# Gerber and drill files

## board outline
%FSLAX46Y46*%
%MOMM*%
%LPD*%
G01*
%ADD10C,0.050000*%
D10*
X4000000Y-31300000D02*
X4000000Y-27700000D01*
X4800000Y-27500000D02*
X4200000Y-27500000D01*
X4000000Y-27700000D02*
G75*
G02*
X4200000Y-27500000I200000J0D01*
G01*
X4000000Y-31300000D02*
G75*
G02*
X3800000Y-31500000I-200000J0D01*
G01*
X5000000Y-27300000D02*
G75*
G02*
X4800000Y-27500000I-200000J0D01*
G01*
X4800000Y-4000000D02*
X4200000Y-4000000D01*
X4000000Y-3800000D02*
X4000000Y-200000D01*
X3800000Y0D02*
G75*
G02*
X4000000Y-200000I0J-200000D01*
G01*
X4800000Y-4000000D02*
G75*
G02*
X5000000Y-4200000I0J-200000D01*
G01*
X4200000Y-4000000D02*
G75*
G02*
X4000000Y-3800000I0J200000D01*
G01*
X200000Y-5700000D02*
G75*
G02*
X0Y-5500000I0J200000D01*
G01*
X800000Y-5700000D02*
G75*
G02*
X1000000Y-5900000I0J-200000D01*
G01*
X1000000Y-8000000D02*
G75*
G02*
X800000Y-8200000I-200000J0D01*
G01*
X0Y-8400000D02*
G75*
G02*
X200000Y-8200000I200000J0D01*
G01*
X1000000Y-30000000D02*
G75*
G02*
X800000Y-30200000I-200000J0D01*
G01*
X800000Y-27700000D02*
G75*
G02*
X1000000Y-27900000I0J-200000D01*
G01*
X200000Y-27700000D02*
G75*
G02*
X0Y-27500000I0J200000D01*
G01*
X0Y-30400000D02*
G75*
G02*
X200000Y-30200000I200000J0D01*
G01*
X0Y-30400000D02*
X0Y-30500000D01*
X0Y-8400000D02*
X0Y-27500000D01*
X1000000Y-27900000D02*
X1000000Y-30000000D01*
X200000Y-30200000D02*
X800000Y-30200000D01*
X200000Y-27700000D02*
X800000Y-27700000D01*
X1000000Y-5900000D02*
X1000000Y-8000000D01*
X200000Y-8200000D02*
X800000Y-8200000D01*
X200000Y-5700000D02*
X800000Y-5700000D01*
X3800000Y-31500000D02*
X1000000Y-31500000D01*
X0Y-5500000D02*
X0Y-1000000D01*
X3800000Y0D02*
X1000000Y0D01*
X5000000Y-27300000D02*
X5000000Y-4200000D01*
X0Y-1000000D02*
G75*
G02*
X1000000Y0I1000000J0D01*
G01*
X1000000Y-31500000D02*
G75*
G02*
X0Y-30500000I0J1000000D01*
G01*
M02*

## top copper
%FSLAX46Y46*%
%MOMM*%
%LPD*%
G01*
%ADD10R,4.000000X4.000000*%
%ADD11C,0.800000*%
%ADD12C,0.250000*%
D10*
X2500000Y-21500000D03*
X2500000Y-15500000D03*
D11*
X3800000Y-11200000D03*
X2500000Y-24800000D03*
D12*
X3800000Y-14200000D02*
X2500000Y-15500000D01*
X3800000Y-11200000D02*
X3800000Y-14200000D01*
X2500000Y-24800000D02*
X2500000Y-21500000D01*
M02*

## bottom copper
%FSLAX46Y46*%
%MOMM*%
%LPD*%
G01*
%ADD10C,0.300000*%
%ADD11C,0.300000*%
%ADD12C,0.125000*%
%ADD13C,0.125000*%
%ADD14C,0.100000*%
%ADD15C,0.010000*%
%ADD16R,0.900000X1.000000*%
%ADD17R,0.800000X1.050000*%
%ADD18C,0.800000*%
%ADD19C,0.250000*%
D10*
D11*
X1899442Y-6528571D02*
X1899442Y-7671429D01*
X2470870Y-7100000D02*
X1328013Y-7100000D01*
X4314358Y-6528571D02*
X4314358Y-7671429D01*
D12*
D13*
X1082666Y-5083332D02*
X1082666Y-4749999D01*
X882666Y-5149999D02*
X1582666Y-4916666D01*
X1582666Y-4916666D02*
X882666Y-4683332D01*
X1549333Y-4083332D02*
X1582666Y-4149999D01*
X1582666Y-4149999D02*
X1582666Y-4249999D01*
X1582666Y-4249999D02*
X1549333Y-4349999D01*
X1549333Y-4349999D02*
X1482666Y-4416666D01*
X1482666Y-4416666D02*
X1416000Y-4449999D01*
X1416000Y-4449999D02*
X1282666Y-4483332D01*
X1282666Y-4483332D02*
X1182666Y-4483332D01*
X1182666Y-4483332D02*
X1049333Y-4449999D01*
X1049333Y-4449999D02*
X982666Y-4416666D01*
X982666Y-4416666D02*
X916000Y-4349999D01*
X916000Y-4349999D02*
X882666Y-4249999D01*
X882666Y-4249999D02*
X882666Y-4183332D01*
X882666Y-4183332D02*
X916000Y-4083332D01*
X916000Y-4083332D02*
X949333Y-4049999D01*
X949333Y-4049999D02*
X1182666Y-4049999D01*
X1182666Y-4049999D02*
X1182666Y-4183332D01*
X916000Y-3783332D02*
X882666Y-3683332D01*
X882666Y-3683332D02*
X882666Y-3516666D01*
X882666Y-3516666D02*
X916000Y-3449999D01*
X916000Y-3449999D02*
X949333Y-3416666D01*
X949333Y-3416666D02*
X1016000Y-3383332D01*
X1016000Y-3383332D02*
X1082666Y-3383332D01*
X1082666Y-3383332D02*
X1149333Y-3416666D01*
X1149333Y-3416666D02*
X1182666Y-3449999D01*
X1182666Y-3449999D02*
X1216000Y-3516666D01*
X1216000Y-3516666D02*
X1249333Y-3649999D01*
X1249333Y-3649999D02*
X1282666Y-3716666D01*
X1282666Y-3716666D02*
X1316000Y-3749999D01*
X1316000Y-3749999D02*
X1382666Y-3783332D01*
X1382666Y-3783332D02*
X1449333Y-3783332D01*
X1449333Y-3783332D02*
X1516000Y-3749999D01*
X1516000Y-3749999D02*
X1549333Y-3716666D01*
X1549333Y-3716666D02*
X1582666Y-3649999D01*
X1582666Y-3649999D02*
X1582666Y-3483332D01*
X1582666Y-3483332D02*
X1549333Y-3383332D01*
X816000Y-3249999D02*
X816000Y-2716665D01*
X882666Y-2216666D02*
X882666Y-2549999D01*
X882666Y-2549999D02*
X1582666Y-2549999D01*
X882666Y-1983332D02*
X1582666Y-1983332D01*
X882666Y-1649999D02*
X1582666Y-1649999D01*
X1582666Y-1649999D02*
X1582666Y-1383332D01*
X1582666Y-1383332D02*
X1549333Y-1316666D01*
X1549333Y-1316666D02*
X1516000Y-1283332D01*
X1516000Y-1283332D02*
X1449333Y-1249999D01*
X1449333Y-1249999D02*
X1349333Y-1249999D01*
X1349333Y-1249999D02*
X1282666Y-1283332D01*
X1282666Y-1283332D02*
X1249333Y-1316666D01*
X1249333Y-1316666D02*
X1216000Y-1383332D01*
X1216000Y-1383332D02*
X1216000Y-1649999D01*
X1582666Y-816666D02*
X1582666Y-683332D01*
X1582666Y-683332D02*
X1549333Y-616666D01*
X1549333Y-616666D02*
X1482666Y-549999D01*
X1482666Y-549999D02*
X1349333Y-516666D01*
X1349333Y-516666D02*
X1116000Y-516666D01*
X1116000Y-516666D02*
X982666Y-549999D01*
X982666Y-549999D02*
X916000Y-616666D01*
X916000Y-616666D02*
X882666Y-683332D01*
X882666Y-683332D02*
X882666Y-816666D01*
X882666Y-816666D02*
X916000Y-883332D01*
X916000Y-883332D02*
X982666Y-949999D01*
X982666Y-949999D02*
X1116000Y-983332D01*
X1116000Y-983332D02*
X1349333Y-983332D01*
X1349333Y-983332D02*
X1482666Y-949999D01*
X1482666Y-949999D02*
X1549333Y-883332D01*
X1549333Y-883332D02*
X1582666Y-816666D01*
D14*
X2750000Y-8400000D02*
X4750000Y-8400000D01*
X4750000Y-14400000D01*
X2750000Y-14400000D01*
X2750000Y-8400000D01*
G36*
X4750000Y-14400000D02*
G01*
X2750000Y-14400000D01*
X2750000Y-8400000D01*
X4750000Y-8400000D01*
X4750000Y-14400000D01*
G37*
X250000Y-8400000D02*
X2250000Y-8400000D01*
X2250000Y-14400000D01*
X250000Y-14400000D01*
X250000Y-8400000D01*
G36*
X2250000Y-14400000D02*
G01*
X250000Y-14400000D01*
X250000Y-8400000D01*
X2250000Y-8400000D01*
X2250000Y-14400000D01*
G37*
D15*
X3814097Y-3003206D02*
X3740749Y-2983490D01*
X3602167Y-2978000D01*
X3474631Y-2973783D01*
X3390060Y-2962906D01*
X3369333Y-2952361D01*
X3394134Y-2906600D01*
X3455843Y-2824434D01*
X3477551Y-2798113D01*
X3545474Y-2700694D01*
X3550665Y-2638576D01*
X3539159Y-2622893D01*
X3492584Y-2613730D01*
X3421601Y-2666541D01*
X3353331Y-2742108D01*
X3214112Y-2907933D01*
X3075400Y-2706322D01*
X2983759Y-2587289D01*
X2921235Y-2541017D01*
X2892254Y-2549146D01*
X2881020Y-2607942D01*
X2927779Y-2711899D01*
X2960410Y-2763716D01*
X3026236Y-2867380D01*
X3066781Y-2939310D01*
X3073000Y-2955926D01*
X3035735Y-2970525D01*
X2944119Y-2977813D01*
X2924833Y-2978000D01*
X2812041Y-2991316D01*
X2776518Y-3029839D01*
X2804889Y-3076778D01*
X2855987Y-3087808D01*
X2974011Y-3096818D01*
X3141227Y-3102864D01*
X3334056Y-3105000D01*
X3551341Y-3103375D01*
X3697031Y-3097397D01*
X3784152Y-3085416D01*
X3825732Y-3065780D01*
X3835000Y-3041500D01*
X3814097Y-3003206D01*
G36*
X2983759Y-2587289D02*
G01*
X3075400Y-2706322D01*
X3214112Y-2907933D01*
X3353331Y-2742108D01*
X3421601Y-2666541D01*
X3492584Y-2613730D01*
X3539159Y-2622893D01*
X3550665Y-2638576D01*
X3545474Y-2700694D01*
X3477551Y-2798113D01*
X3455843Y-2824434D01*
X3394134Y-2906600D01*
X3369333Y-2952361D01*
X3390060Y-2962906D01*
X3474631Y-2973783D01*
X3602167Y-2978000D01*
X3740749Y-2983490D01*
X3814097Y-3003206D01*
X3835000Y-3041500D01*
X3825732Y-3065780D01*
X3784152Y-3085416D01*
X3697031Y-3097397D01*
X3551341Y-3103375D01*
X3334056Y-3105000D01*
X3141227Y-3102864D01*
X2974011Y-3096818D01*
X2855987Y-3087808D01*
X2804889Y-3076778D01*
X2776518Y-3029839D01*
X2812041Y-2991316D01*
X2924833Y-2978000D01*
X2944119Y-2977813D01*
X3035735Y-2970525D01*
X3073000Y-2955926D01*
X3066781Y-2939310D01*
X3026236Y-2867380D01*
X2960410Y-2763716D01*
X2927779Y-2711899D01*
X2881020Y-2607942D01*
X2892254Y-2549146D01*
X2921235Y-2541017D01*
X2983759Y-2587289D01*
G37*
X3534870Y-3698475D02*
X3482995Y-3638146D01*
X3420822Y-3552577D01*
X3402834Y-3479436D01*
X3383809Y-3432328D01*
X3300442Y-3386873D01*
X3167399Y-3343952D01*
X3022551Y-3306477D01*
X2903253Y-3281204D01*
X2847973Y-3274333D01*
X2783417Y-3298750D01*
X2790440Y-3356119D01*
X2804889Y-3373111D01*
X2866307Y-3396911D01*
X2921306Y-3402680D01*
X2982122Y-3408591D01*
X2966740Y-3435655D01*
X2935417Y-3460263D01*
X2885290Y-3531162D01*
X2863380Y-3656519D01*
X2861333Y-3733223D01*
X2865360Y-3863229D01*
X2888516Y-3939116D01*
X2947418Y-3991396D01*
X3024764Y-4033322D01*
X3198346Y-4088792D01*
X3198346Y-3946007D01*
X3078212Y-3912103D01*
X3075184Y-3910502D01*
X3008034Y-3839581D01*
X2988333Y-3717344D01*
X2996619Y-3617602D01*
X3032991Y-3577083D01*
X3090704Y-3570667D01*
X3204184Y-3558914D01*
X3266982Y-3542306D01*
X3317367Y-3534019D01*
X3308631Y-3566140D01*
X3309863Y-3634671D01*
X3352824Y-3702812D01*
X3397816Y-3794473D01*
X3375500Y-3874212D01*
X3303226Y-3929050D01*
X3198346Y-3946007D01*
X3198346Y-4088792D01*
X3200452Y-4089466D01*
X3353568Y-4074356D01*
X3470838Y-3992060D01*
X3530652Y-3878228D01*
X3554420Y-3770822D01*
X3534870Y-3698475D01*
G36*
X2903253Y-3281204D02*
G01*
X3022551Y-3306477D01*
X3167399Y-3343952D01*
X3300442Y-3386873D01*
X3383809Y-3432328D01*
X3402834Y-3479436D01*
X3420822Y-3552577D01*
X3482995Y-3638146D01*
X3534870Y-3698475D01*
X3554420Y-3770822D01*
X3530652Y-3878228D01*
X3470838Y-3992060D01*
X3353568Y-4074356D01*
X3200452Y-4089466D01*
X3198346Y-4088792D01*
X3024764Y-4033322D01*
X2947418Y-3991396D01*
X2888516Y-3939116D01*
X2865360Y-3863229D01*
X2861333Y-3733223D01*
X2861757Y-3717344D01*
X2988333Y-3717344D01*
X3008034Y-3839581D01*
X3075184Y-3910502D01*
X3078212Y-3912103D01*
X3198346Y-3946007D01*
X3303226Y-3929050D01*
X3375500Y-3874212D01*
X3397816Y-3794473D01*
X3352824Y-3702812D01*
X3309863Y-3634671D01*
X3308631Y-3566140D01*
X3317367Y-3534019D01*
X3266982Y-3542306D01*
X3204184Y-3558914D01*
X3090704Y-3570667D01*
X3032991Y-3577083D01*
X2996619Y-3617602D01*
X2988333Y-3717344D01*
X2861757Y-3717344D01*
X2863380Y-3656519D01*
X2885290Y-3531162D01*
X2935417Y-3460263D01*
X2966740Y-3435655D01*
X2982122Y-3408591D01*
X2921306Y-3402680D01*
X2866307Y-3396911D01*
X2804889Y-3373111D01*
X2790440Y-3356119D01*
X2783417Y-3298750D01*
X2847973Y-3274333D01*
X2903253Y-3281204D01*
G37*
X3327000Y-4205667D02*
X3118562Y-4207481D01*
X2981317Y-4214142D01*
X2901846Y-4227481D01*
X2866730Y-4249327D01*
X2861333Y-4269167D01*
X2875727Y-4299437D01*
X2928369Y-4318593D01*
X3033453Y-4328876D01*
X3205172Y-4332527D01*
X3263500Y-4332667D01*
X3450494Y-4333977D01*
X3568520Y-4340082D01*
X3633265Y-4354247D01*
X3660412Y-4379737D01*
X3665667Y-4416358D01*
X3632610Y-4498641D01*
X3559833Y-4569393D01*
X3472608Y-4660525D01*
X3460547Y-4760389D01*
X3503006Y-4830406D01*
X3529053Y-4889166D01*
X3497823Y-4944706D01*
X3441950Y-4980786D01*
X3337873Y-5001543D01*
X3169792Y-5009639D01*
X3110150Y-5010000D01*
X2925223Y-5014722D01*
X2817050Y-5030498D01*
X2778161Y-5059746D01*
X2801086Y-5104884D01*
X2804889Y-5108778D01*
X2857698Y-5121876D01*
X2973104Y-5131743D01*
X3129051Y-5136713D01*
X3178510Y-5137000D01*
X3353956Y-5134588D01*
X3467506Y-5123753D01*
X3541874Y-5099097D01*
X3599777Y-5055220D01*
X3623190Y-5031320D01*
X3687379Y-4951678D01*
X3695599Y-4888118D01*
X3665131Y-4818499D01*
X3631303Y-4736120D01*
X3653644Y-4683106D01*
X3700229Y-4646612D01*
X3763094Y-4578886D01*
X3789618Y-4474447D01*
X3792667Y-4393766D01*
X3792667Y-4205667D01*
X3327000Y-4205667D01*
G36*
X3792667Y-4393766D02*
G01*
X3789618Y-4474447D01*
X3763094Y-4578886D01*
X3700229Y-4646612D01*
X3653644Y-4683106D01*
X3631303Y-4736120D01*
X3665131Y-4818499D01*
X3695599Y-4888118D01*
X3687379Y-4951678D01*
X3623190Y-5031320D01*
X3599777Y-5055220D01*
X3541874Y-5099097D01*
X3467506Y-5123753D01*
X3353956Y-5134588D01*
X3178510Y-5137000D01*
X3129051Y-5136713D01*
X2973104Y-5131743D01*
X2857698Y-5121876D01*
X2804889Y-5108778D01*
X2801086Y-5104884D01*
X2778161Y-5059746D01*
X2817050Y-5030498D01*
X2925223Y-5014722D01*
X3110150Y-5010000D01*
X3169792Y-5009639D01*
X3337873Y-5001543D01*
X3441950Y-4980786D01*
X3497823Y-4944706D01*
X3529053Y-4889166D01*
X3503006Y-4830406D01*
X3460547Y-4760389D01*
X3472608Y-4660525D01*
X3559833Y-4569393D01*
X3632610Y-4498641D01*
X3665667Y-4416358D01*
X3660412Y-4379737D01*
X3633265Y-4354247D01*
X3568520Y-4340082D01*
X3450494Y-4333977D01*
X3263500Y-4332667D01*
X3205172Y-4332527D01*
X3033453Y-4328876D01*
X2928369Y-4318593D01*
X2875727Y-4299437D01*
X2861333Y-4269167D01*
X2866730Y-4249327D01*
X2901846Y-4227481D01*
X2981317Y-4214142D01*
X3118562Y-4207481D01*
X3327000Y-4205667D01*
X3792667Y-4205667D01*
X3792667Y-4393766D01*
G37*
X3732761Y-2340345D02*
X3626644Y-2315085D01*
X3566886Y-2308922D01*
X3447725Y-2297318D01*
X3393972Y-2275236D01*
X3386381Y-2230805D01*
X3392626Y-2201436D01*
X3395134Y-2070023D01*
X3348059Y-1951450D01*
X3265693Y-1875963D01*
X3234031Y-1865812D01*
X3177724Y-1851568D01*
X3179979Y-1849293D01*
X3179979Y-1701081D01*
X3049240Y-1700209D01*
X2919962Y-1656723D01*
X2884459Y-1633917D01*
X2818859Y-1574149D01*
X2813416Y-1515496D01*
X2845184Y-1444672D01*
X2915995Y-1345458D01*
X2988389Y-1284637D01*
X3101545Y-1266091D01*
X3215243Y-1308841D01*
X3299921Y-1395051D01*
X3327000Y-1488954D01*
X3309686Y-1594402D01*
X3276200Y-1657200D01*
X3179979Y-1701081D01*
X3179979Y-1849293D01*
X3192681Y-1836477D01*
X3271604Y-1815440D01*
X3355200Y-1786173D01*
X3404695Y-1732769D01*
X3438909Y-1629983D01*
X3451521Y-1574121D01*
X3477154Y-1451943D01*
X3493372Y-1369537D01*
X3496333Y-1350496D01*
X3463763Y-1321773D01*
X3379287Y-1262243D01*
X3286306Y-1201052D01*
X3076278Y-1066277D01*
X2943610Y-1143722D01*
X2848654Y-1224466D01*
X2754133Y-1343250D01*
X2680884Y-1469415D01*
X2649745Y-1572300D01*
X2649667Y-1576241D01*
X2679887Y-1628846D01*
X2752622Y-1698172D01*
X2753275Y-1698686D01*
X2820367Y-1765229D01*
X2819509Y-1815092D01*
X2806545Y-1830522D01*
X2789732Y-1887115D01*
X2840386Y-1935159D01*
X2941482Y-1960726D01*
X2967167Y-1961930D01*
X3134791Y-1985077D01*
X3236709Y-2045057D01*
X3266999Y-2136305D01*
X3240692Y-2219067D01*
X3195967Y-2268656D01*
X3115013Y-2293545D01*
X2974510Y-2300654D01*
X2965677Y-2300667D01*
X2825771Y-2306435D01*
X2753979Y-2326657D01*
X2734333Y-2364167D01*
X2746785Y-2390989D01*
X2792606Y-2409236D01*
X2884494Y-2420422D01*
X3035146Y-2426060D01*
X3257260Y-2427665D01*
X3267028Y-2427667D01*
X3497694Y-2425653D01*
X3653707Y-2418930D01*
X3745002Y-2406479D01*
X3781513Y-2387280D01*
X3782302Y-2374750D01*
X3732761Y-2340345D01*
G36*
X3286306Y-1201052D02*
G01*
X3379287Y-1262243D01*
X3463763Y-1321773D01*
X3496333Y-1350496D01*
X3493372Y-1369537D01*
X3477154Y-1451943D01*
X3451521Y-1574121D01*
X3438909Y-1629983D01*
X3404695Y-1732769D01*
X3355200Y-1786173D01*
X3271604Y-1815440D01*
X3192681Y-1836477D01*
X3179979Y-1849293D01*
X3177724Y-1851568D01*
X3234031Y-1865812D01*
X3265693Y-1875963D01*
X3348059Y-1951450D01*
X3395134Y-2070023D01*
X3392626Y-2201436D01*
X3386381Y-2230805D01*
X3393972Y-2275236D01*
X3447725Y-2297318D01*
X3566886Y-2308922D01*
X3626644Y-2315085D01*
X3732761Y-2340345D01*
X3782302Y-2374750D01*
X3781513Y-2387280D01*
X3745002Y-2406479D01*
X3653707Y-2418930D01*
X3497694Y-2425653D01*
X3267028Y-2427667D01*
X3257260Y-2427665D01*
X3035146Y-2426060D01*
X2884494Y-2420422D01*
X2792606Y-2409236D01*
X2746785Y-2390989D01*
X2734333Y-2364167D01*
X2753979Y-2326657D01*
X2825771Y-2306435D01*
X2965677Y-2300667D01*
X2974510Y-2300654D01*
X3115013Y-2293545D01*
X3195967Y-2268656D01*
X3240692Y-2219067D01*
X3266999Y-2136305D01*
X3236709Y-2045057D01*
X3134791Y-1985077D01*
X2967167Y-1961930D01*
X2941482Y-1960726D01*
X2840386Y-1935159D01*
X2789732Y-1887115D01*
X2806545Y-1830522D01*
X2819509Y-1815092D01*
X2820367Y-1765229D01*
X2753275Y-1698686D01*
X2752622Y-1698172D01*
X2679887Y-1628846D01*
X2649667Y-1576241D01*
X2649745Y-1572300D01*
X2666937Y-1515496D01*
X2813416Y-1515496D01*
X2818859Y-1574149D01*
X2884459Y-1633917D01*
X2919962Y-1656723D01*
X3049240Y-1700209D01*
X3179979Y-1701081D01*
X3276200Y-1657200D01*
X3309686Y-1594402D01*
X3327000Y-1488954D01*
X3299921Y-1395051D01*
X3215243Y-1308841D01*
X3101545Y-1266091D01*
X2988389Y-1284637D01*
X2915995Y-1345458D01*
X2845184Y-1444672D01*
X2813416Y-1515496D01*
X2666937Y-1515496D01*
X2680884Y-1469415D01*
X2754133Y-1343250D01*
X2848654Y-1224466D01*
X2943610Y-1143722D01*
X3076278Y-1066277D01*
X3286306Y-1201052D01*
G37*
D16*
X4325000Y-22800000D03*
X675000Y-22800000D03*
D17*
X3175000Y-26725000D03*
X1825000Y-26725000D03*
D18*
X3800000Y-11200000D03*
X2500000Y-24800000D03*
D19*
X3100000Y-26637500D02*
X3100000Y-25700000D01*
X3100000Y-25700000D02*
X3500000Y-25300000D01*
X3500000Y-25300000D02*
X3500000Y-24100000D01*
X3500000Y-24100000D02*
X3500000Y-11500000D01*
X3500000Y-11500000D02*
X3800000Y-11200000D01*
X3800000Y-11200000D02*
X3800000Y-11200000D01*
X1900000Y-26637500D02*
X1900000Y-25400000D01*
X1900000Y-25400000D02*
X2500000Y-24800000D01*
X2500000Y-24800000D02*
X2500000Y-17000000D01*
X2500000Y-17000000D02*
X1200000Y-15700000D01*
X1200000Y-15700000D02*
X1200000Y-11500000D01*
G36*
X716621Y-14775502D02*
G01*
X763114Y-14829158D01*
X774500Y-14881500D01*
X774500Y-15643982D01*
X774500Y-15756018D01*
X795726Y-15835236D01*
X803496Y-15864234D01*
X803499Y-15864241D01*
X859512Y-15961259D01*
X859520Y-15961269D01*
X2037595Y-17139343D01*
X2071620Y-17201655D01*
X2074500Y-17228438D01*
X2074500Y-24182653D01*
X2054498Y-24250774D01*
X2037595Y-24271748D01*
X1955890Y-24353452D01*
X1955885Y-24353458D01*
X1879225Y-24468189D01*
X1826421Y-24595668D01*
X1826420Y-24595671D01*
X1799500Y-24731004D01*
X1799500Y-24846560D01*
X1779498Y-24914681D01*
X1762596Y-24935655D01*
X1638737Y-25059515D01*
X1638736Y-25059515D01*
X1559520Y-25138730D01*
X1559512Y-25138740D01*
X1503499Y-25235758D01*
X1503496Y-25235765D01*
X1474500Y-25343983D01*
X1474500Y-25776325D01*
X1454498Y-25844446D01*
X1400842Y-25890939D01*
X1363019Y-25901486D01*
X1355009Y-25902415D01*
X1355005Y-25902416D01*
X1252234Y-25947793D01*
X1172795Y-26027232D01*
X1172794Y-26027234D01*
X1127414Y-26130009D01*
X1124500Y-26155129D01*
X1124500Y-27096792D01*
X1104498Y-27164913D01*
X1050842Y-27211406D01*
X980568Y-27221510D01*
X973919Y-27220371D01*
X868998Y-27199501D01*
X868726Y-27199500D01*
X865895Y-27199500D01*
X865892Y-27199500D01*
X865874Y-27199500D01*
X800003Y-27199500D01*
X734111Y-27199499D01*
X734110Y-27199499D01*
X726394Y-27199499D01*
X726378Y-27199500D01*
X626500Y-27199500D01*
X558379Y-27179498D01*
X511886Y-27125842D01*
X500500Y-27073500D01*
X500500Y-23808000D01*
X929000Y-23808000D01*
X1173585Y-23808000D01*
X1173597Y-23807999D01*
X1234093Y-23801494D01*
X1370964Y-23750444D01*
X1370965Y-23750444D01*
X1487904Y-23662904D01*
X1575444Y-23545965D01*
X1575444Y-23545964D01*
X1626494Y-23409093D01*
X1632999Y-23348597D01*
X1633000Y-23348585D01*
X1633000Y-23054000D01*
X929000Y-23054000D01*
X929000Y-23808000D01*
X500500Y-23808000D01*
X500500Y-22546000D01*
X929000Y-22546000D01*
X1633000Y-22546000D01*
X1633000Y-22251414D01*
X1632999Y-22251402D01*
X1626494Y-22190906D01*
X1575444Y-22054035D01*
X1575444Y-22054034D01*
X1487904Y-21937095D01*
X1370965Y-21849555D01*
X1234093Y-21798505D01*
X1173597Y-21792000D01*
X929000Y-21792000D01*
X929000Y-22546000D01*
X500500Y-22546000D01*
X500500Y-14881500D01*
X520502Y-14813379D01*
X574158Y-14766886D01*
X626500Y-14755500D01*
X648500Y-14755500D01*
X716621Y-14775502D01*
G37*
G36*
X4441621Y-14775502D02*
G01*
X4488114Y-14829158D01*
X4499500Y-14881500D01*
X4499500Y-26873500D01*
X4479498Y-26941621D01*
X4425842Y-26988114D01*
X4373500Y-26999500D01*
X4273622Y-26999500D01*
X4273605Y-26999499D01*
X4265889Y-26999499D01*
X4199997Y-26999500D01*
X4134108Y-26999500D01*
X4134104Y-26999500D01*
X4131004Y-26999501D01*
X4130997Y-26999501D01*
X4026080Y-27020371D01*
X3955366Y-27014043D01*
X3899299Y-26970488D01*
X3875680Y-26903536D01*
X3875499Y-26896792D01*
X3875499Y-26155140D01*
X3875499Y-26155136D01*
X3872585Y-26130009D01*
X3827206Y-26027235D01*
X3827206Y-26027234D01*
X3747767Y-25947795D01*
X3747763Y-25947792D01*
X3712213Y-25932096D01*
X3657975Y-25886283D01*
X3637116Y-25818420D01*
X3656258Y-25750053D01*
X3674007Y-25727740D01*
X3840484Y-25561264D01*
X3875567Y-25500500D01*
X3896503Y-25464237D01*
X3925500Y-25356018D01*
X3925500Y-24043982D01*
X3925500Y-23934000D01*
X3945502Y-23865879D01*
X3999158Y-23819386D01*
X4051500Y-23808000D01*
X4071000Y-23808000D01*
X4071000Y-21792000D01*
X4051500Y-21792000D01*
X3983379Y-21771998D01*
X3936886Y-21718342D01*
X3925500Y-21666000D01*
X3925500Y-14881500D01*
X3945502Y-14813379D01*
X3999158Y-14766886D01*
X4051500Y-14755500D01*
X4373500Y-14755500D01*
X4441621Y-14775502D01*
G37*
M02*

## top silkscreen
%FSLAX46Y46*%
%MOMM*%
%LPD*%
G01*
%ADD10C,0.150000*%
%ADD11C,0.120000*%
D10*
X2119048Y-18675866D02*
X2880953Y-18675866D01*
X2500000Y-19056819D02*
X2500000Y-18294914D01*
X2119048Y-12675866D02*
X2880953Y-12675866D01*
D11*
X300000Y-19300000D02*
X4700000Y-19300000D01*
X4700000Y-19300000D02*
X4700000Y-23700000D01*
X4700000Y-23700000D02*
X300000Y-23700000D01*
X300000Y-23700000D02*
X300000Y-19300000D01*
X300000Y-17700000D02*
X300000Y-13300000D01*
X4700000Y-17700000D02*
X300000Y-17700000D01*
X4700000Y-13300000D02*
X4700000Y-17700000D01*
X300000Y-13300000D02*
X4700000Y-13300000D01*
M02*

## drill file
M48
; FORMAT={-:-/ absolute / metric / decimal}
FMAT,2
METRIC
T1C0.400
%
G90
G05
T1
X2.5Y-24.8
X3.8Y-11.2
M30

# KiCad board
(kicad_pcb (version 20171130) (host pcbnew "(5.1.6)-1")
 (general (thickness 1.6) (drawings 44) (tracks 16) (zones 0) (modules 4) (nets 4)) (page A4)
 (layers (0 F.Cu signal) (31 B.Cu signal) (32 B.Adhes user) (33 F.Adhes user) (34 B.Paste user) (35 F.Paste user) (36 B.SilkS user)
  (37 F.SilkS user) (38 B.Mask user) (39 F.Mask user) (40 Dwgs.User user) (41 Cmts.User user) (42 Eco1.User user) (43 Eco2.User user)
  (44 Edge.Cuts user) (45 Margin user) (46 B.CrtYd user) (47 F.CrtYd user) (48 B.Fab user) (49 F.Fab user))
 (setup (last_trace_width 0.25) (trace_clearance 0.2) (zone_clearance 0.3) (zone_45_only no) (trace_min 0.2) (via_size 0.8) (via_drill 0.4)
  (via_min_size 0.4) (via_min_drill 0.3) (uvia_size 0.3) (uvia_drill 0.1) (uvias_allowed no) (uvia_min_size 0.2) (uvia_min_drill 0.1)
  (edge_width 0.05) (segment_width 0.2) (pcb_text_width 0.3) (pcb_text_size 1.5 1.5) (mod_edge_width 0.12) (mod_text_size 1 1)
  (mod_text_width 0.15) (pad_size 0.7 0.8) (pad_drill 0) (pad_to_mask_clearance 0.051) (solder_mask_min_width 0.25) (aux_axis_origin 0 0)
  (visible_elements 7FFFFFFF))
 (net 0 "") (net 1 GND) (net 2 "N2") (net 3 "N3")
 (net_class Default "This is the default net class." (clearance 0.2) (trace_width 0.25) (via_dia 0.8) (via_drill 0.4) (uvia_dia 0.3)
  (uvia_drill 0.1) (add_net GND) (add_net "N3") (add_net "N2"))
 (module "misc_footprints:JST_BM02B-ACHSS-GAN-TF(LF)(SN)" (layer B.Cu) (at 2.5 24.75)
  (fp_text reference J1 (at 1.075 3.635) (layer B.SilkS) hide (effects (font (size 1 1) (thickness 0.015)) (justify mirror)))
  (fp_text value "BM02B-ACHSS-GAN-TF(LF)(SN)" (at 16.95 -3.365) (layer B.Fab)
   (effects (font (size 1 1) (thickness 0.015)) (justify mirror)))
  (pad S2 smd rect (at 1.825 -1.95) (size 0.9 1) (layers B.Cu B.Paste B.Mask) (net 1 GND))
  (pad S1 smd rect (at -1.825 -1.95) (size 0.9 1) (layers B.Cu B.Paste B.Mask) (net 1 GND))
  (pad 2 smd rect (at 0.675 1.975) (size 0.8 1.05) (layers B.Cu B.Paste B.Mask) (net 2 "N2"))
  (pad 1 smd rect (at -0.675 1.975) (size 0.8 1.05) (layers B.Cu B.Paste B.Mask) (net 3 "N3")))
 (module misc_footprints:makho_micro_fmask (layer B.Cu) (at 3.3 3.1 90)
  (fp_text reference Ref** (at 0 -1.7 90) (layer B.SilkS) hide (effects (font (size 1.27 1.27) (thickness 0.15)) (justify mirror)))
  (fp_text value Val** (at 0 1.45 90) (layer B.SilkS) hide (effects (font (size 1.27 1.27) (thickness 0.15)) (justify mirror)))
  (fp_poly
   (pts (xy 0.096794 0.514097) (xy 0.11651 0.440749) (xy 0.122 0.302167) (xy 0.126217 0.174631) (xy 0.137094 0.09006) (xy 0.147639 0.069333)
    (xy 0.1934 0.094134) (xy 0.275566 0.155843) (xy 0.301887 0.177551) (xy 0.399306 0.245474) (xy 0.461424 0.250665) (xy 0.477107 0.239159)
    (xy 0.48627 0.192584) (xy 0.433459 0.121601) (xy 0.357892 0.053331) (xy 0.192067 -0.085888) (xy 0.393678 -0.2246)
    (xy 0.512711 -0.316241) (xy 0.558983 -0.378765) (xy 0.550854 -0.407746) (xy 0.492058 -0.41898) (xy 0.388101 -0.372221)
    (xy 0.336284 -0.33959) (xy 0.23262 -0.273764) (xy 0.16069 -0.233219) (xy 0.144074 -0.227) (xy 0.129475 -0.264265)
    (xy 0.122187 -0.355881) (xy 0.122 -0.375167) (xy 0.108684 -0.487959) (xy 0.070161 -0.523482) (xy 0.023222 -0.495111)
    (xy 0.012192 -0.444013) (xy 0.003182 -0.325989) (xy -0.002864 -0.158773) (xy -0.005 0.034056) (xy -0.003375 0.251341)
    (xy 0.002603 0.397031) (xy 0.014584 0.484152) (xy 0.03422 0.525732) (xy 0.0585 0.535) (xy 0.096794 0.514097))
   (layer B.Cu) (width 0.01))
  (fp_poly
   (pts (xy -0.598475 0.23487) (xy -0.538146 0.182995) (xy -0.452577 0.120822) (xy -0.379436 0.102834) (xy -0.332328 0.083809)
    (xy -0.286873 0.000442) (xy -0.243952 -0.132601) (xy -0.206477 -0.277449) (xy -0.181204 -0.396747) (xy -0.174333 -0.452027)
    (xy -0.19875 -0.516583) (xy -0.256119 -0.50956) (xy -0.273111 -0.495111) (xy -0.296911 -0.433693) (xy -0.30268 -0.378694)
    (xy -0.308591 -0.317878) (xy -0.335655 -0.33326) (xy -0.360263 -0.364583) (xy -0.431162 -0.41471) (xy -0.556519 -0.43662)
    (xy -0.633223 -0.438667) (xy -0.763229 -0.43464) (xy -0.839116 -0.411484) (xy -0.891396 -0.352582) (xy -0.933322 -0.275236)
    (xy -0.988792 -0.101654) (xy -0.846007 -0.101654) (xy -0.812103 -0.221788) (xy -0.810502 -0.224816) (xy -0.739581 -0.291966)
    (xy -0.617344 -0.311667) (xy -0.517602 -0.303381) (xy -0.477083 -0.267009) (xy -0.470667 -0.209296) (xy -0.458914 -0.095816)
    (xy -0.442306 -0.033018) (xy -0.434019 0.017367) (xy -0.46614 0.008631) (xy -0.534671 0.009863) (xy -0.602812 0.052824)
    (xy -0.694473 0.097816) (xy -0.774212 0.0755) (xy -0.82905 0.003226) (xy -0.846007 -0.101654) (xy -0.988792 -0.101654)
    (xy -0.989466 -0.099548) (xy -0.974356 0.053568) (xy -0.89206 0.170838) (xy -0.778228 0.230652) (xy -0.670822 0.25442)
    (xy -0.598475 0.23487))
   (layer B.Cu) (width 0.01))
  (fp_poly
   (pts (xy -1.105667 0.027) (xy -1.107481 -0.181438) (xy -1.114142 -0.318683) (xy -1.127481 -0.398154) (xy -1.149327 -0.43327)
    (xy -1.169167 -0.438667) (xy -1.199437 -0.424273) (xy -1.218593 -0.371631) (xy -1.228876 -0.266547) (xy -1.232527 -0.094828)
    (xy -1.232667 -0.0365) (xy -1.233977 0.150494) (xy -1.240082 0.26852) (xy -1.254247 0.333265) (xy -1.279737 0.360412)
    (xy -1.316358 0.365667) (xy -1.398641 0.33261) (xy -1.469393 0.259833) (xy -1.560525 0.172608) (xy -1.660389 0.160547)
    (xy -1.730406 0.203006) (xy -1.789166 0.229053) (xy -1.844706 0.197823) (xy -1.880786 0.14195) (xy -1.901543 0.037873)
    (xy -1.909639 -0.130208) (xy -1.91 -0.18985) (xy -1.914722 -0.374777) (xy -1.930498 -0.48295) (xy -1.959746 -0.521839)
    (xy -2.004884 -0.498914) (xy -2.008778 -0.495111) (xy -2.021876 -0.442302) (xy -2.031743 -0.326896) (xy -2.036713 -0.170949)
    (xy -2.037 -0.12149) (xy -2.034588 0.053956) (xy -2.023753 0.167506) (xy -1.999097 0.241874) (xy -1.95522 0.299777)
    (xy -1.93132 0.32319) (xy -1.851678 0.387379) (xy -1.788118 0.395599) (xy -1.718499 0.365131) (xy -1.63612 0.331303)
    (xy -1.583106 0.353644) (xy -1.546612 0.400229) (xy -1.478886 0.463094) (xy -1.374447 0.489618) (xy -1.293766 0.492667)
    (xy -1.105667 0.492667) (xy -1.105667 0.027))
   (layer B.Cu) (width 0.01))
  (fp_poly
   (pts (xy 0.759655 0.432761) (xy 0.784915 0.326644) (xy 0.791078 0.266886) (xy 0.802682 0.147725) (xy 0.824764 0.093972)
    (xy 0.869195 0.086381) (xy 0.898564 0.092626) (xy 1.029977 0.095134) (xy 1.14855 0.048059) (xy 1.224037 -0.034307)
    (xy 1.234188 -0.065969) (xy 1.248432 -0.122276) (xy 1.250707 -0.120021) (xy 1.398919 -0.120021) (xy 1.399791 -0.25076)
    (xy 1.443277 -0.380038) (xy 1.466083 -0.415541) (xy 1.525851 -0.481141) (xy 1.584504 -0.486584) (xy 1.655328 -0.454816)
    (xy 1.754542 -0.384005) (xy 1.815363 -0.311611) (xy 1.833909 -0.198455) (xy 1.791159 -0.084757) (xy 1.704949 -0.000079)
    (xy 1.611046 0.027) (xy 1.505598 0.009686) (xy 1.4428 -0.0238) (xy 1.398919 -0.120021) (xy 1.250707 -0.120021) (xy 1.263523 -0.107319)
    (xy 1.28456 -0.028396) (xy 1.313827 0.0552) (xy 1.367231 0.104695) (xy 1.470017 0.138909) (xy 1.525879 0.151521) (xy 1.648057 0.177154)
    (xy 1.730463 0.193372) (xy 1.749504 0.196333) (xy 1.778227 0.163763) (xy 1.837757 0.079287) (xy 1.898948 -0.013694)
    (xy 2.033723 -0.223722) (xy 1.956278 -0.35639) (xy 1.875534 -0.451346) (xy 1.75675 -0.545867) (xy 1.630585 -0.619116)
    (xy 1.5277 -0.650255) (xy 1.523759 -0.650333) (xy 1.471154 -0.620113) (xy 1.401828 -0.547378) (xy 1.401314 -0.546725)
    (xy 1.334771 -0.479633) (xy 1.284908 -0.480491) (xy 1.269478 -0.493455) (xy 1.212885 -0.510268) (xy 1.164841 -0.459614)
    (xy 1.139274 -0.358518) (xy 1.13807 -0.332833) (xy 1.114923 -0.165209) (xy 1.054943 -0.063291) (xy 0.963695 -0.033001)
    (xy 0.880933 -0.059308) (xy 0.831344 -0.104033) (xy 0.806455 -0.184987) (xy 0.799346 -0.32549) (xy 0.799333 -0.334323)
    (xy 0.793565 -0.474229) (xy 0.773343 -0.546021) (xy 0.735833 -0.565667) (xy 0.709011 -0.553215) (xy 0.690764 -0.507394)
    (xy 0.679578 -0.415506) (xy 0.67394 -0.264854) (xy 0.672335 -0.04274) (xy 0.672333 -0.032972) (xy 0.674347 0.197694)
    (xy 0.68107 0.353707) (xy 0.693521 0.445002) (xy 0.71272 0.481513) (xy 0.72525 0.482302) (xy 0.759655 0.432761))
   (layer B.Cu) (width 0.01)))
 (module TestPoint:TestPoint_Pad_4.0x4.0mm (layer F.Cu) (at 2.5 21.5)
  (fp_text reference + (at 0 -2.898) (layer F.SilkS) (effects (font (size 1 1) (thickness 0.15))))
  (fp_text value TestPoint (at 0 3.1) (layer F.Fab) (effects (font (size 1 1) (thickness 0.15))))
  (fp_line (start -2.2 -2.2) (end 2.2 -2.2) (layer F.SilkS) (width 0.12))
  (fp_line (start 2.2 -2.2) (end 2.2 2.2) (layer F.SilkS) (width 0.12))
  (fp_line (start 2.2 2.2) (end -2.2 2.2) (layer F.SilkS) (width 0.12))
  (fp_line (start -2.2 2.2) (end -2.2 -2.2) (layer F.SilkS) (width 0.12))
  (pad 1 smd rect (at 0 0) (size 4 4) (layers F.Cu F.Mask) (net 3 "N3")))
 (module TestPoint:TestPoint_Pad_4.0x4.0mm (layer F.Cu) (at 2.5 15.5)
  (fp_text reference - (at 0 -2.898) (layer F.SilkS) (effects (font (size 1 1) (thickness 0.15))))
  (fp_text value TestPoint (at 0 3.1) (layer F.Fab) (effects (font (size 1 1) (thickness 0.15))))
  (fp_line (start -2.2 2.2) (end -2.2 -2.2) (layer F.SilkS) (width 0.12))
  (fp_line (start 2.2 2.2) (end -2.2 2.2) (layer F.SilkS) (width 0.12))
  (fp_line (start 2.2 -2.2) (end 2.2 2.2) (layer F.SilkS) (width 0.12))
  (fp_line (start -2.2 -2.2) (end 2.2 -2.2) (layer F.SilkS) (width 0.12))
  (pad 1 smd rect (at 0 0) (size 4 4) (layers F.Cu F.Mask) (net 2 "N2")))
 (gr_line (start 4 31.3) (end 4 27.7) (layer Edge.Cuts) (width 0.05))
 (gr_line (start 4.8 27.5) (end 4.2 27.5) (layer Edge.Cuts) (width 0.05))
 (gr_arc (start 4.2 27.7) (end 4.2 27.5) (angle -90) (layer Edge.Cuts) (width 0.05))
 (gr_arc (start 3.8 31.3) (end 3.8 31.5) (angle -90) (layer Edge.Cuts) (width 0.05))
 (gr_arc (start 4.8 27.3) (end 4.8 27.5) (angle -90) (layer Edge.Cuts) (width 0.05))
 (gr_line (start 4.8 4) (end 4.2 4) (layer Edge.Cuts) (width 0.05))
 (gr_line (start 4 3.8) (end 4 0.2) (layer Edge.Cuts) (width 0.05))
 (gr_arc (start 3.8 0.2) (end 4 0.2) (angle -90) (layer Edge.Cuts) (width 0.05))
 (gr_arc (start 4.8 4.2) (end 5 4.2) (angle -90) (layer Edge.Cuts) (width 0.05))
 (gr_arc (start 4.2 3.8) (end 4 3.8) (angle -90) (layer Edge.Cuts) (width 0.05))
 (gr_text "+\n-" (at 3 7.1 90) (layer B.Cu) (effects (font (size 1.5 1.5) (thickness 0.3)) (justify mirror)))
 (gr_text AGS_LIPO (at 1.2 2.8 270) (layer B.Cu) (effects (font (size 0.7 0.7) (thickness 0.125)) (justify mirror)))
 (gr_arc (start 0.2 5.5) (end 0 5.5) (angle -90) (layer Edge.Cuts) (width 0.05))
 (gr_arc (start 0.8 5.9) (end 1 5.9) (angle -90) (layer Edge.Cuts) (width 0.05))
 (gr_arc (start 0.8 8) (end 0.8 8.2) (angle -90) (layer Edge.Cuts) (width 0.05))
 (gr_arc (start 0.2 8.4) (end 0.2 8.2) (angle -90) (layer Edge.Cuts) (width 0.05))
 (gr_arc (start 0.8 30) (end 0.8 30.2) (angle -90) (layer Edge.Cuts) (width 0.05))
 (gr_arc (start 0.8 27.9) (end 1 27.9) (angle -90) (layer Edge.Cuts) (width 0.05))
 (gr_arc (start 0.2 27.5) (end 0 27.5) (angle -90) (layer Edge.Cuts) (width 0.05))
 (gr_arc (start 0.2 30.4) (end 0.2 30.2) (angle -90) (layer Edge.Cuts) (width 0.05))
 (gr_line (start 0 30.4) (end 0 30.5) (layer Edge.Cuts) (width 0.05))
 (gr_line (start 0 8.4) (end 0 27.5) (layer Edge.Cuts) (width 0.05))
 (gr_line (start 1 27.9) (end 1 30) (layer Edge.Cuts) (width 0.05))
 (gr_line (start 0.2 30.2) (end 0.8 30.2) (layer Edge.Cuts) (width 0.05))
 (gr_line (start 0.2 27.7) (end 0.8 27.7) (layer Edge.Cuts) (width 0.05))
 (gr_line (start 1 5.9) (end 1 8) (layer Edge.Cuts) (width 0.05))
 (gr_line (start 0.2 8.2) (end 0.8 8.2) (layer Edge.Cuts) (width 0.05))
 (gr_line (start 0.2 5.7) (end 0.8 5.7) (layer Edge.Cuts) (width 0.05))
 (gr_poly (pts (xy 2.75 8.4) (xy 4.75 8.4) (xy 4.75 14.4) (xy 2.75 14.4)) (layer B.Cu) (width 0.1))
 (gr_poly (pts (xy 0.25 8.4) (xy 2.25 8.4) (xy 2.25 14.4) (xy 0.25 14.4)) (layer B.Cu) (width 0.1))
 (gr_line (start 3.8 31.5) (end 1 31.5) (layer Edge.Cuts) (width 0.05))
 (gr_line (start 0 5.5) (end 0 1) (layer Edge.Cuts) (width 0.05))
 (gr_line (start 3.8 0) (end 1 0) (layer Edge.Cuts) (width 0.05))
 (gr_line (start 5 27.3) (end 5 4.2) (layer Edge.Cuts) (width 0.05))
 (gr_arc (start 1 1) (end 1 0) (angle -90) (layer Edge.Cuts) (width 0.05))
 (gr_arc (start 1 30.5) (end 0 30.5) (angle -90) (layer Edge.Cuts) (width 0.05))
 (segment (start 3.1 26.6375) (end 3.1 25.7) (width 0.25) (layer B.Cu) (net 2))
 (segment (start 3.1 25.7) (end 3.5 25.3) (width 0.25) (layer B.Cu) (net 2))
 (segment (start 3.5 25.3) (end 3.5 24.1) (width 0.25) (layer B.Cu) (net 2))
 (segment (start 3.5 24.1) (end 3.5 11.5) (width 0.25) (layer B.Cu) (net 2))
 (segment (start 3.5 11.5) (end 3.8 11.2) (width 0.25) (layer B.Cu) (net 2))
 (segment (start 3.8 11.2) (end 3.8 11.2) (width 0.25) (layer B.Cu) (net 2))
 (via (at 3.8 11.2) (size 0.8) (drill 0.4) (layers F.Cu B.Cu) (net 2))
 (segment (start 3.8 14.2) (end 2.5 15.5) (width 0.25) (layer F.Cu) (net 2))
 (segment (start 3.8 11.2) (end 3.8 14.2) (width 0.25) (layer F.Cu) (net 2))
 (via (at 2.5 24.8) (size 0.8) (drill 0.4) (layers F.Cu B.Cu) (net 3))
 (segment (start 1.9 26.6375) (end 1.9 25.4) (width 0.25) (layer B.Cu) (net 3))
 (segment (start 1.9 25.4) (end 2.5 24.8) (width 0.25) (layer B.Cu) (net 3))
 (segment (start 2.5 24.8) (end 2.5 21.5) (width 0.25) (layer F.Cu) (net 3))
 (segment (start 2.5 24.8) (end 2.5 17) (width 0.25) (layer B.Cu) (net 3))
 (segment (start 2.5 17) (end 1.2 15.7) (width 0.25) (layer B.Cu) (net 3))
 (segment (start 1.2 15.7) (end 1.2 11.5) (width 0.25) (layer B.Cu) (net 3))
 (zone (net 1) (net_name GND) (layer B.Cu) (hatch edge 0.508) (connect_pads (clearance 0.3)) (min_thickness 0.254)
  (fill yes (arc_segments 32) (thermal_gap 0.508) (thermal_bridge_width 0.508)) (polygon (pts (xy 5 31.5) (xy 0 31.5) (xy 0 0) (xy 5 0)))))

